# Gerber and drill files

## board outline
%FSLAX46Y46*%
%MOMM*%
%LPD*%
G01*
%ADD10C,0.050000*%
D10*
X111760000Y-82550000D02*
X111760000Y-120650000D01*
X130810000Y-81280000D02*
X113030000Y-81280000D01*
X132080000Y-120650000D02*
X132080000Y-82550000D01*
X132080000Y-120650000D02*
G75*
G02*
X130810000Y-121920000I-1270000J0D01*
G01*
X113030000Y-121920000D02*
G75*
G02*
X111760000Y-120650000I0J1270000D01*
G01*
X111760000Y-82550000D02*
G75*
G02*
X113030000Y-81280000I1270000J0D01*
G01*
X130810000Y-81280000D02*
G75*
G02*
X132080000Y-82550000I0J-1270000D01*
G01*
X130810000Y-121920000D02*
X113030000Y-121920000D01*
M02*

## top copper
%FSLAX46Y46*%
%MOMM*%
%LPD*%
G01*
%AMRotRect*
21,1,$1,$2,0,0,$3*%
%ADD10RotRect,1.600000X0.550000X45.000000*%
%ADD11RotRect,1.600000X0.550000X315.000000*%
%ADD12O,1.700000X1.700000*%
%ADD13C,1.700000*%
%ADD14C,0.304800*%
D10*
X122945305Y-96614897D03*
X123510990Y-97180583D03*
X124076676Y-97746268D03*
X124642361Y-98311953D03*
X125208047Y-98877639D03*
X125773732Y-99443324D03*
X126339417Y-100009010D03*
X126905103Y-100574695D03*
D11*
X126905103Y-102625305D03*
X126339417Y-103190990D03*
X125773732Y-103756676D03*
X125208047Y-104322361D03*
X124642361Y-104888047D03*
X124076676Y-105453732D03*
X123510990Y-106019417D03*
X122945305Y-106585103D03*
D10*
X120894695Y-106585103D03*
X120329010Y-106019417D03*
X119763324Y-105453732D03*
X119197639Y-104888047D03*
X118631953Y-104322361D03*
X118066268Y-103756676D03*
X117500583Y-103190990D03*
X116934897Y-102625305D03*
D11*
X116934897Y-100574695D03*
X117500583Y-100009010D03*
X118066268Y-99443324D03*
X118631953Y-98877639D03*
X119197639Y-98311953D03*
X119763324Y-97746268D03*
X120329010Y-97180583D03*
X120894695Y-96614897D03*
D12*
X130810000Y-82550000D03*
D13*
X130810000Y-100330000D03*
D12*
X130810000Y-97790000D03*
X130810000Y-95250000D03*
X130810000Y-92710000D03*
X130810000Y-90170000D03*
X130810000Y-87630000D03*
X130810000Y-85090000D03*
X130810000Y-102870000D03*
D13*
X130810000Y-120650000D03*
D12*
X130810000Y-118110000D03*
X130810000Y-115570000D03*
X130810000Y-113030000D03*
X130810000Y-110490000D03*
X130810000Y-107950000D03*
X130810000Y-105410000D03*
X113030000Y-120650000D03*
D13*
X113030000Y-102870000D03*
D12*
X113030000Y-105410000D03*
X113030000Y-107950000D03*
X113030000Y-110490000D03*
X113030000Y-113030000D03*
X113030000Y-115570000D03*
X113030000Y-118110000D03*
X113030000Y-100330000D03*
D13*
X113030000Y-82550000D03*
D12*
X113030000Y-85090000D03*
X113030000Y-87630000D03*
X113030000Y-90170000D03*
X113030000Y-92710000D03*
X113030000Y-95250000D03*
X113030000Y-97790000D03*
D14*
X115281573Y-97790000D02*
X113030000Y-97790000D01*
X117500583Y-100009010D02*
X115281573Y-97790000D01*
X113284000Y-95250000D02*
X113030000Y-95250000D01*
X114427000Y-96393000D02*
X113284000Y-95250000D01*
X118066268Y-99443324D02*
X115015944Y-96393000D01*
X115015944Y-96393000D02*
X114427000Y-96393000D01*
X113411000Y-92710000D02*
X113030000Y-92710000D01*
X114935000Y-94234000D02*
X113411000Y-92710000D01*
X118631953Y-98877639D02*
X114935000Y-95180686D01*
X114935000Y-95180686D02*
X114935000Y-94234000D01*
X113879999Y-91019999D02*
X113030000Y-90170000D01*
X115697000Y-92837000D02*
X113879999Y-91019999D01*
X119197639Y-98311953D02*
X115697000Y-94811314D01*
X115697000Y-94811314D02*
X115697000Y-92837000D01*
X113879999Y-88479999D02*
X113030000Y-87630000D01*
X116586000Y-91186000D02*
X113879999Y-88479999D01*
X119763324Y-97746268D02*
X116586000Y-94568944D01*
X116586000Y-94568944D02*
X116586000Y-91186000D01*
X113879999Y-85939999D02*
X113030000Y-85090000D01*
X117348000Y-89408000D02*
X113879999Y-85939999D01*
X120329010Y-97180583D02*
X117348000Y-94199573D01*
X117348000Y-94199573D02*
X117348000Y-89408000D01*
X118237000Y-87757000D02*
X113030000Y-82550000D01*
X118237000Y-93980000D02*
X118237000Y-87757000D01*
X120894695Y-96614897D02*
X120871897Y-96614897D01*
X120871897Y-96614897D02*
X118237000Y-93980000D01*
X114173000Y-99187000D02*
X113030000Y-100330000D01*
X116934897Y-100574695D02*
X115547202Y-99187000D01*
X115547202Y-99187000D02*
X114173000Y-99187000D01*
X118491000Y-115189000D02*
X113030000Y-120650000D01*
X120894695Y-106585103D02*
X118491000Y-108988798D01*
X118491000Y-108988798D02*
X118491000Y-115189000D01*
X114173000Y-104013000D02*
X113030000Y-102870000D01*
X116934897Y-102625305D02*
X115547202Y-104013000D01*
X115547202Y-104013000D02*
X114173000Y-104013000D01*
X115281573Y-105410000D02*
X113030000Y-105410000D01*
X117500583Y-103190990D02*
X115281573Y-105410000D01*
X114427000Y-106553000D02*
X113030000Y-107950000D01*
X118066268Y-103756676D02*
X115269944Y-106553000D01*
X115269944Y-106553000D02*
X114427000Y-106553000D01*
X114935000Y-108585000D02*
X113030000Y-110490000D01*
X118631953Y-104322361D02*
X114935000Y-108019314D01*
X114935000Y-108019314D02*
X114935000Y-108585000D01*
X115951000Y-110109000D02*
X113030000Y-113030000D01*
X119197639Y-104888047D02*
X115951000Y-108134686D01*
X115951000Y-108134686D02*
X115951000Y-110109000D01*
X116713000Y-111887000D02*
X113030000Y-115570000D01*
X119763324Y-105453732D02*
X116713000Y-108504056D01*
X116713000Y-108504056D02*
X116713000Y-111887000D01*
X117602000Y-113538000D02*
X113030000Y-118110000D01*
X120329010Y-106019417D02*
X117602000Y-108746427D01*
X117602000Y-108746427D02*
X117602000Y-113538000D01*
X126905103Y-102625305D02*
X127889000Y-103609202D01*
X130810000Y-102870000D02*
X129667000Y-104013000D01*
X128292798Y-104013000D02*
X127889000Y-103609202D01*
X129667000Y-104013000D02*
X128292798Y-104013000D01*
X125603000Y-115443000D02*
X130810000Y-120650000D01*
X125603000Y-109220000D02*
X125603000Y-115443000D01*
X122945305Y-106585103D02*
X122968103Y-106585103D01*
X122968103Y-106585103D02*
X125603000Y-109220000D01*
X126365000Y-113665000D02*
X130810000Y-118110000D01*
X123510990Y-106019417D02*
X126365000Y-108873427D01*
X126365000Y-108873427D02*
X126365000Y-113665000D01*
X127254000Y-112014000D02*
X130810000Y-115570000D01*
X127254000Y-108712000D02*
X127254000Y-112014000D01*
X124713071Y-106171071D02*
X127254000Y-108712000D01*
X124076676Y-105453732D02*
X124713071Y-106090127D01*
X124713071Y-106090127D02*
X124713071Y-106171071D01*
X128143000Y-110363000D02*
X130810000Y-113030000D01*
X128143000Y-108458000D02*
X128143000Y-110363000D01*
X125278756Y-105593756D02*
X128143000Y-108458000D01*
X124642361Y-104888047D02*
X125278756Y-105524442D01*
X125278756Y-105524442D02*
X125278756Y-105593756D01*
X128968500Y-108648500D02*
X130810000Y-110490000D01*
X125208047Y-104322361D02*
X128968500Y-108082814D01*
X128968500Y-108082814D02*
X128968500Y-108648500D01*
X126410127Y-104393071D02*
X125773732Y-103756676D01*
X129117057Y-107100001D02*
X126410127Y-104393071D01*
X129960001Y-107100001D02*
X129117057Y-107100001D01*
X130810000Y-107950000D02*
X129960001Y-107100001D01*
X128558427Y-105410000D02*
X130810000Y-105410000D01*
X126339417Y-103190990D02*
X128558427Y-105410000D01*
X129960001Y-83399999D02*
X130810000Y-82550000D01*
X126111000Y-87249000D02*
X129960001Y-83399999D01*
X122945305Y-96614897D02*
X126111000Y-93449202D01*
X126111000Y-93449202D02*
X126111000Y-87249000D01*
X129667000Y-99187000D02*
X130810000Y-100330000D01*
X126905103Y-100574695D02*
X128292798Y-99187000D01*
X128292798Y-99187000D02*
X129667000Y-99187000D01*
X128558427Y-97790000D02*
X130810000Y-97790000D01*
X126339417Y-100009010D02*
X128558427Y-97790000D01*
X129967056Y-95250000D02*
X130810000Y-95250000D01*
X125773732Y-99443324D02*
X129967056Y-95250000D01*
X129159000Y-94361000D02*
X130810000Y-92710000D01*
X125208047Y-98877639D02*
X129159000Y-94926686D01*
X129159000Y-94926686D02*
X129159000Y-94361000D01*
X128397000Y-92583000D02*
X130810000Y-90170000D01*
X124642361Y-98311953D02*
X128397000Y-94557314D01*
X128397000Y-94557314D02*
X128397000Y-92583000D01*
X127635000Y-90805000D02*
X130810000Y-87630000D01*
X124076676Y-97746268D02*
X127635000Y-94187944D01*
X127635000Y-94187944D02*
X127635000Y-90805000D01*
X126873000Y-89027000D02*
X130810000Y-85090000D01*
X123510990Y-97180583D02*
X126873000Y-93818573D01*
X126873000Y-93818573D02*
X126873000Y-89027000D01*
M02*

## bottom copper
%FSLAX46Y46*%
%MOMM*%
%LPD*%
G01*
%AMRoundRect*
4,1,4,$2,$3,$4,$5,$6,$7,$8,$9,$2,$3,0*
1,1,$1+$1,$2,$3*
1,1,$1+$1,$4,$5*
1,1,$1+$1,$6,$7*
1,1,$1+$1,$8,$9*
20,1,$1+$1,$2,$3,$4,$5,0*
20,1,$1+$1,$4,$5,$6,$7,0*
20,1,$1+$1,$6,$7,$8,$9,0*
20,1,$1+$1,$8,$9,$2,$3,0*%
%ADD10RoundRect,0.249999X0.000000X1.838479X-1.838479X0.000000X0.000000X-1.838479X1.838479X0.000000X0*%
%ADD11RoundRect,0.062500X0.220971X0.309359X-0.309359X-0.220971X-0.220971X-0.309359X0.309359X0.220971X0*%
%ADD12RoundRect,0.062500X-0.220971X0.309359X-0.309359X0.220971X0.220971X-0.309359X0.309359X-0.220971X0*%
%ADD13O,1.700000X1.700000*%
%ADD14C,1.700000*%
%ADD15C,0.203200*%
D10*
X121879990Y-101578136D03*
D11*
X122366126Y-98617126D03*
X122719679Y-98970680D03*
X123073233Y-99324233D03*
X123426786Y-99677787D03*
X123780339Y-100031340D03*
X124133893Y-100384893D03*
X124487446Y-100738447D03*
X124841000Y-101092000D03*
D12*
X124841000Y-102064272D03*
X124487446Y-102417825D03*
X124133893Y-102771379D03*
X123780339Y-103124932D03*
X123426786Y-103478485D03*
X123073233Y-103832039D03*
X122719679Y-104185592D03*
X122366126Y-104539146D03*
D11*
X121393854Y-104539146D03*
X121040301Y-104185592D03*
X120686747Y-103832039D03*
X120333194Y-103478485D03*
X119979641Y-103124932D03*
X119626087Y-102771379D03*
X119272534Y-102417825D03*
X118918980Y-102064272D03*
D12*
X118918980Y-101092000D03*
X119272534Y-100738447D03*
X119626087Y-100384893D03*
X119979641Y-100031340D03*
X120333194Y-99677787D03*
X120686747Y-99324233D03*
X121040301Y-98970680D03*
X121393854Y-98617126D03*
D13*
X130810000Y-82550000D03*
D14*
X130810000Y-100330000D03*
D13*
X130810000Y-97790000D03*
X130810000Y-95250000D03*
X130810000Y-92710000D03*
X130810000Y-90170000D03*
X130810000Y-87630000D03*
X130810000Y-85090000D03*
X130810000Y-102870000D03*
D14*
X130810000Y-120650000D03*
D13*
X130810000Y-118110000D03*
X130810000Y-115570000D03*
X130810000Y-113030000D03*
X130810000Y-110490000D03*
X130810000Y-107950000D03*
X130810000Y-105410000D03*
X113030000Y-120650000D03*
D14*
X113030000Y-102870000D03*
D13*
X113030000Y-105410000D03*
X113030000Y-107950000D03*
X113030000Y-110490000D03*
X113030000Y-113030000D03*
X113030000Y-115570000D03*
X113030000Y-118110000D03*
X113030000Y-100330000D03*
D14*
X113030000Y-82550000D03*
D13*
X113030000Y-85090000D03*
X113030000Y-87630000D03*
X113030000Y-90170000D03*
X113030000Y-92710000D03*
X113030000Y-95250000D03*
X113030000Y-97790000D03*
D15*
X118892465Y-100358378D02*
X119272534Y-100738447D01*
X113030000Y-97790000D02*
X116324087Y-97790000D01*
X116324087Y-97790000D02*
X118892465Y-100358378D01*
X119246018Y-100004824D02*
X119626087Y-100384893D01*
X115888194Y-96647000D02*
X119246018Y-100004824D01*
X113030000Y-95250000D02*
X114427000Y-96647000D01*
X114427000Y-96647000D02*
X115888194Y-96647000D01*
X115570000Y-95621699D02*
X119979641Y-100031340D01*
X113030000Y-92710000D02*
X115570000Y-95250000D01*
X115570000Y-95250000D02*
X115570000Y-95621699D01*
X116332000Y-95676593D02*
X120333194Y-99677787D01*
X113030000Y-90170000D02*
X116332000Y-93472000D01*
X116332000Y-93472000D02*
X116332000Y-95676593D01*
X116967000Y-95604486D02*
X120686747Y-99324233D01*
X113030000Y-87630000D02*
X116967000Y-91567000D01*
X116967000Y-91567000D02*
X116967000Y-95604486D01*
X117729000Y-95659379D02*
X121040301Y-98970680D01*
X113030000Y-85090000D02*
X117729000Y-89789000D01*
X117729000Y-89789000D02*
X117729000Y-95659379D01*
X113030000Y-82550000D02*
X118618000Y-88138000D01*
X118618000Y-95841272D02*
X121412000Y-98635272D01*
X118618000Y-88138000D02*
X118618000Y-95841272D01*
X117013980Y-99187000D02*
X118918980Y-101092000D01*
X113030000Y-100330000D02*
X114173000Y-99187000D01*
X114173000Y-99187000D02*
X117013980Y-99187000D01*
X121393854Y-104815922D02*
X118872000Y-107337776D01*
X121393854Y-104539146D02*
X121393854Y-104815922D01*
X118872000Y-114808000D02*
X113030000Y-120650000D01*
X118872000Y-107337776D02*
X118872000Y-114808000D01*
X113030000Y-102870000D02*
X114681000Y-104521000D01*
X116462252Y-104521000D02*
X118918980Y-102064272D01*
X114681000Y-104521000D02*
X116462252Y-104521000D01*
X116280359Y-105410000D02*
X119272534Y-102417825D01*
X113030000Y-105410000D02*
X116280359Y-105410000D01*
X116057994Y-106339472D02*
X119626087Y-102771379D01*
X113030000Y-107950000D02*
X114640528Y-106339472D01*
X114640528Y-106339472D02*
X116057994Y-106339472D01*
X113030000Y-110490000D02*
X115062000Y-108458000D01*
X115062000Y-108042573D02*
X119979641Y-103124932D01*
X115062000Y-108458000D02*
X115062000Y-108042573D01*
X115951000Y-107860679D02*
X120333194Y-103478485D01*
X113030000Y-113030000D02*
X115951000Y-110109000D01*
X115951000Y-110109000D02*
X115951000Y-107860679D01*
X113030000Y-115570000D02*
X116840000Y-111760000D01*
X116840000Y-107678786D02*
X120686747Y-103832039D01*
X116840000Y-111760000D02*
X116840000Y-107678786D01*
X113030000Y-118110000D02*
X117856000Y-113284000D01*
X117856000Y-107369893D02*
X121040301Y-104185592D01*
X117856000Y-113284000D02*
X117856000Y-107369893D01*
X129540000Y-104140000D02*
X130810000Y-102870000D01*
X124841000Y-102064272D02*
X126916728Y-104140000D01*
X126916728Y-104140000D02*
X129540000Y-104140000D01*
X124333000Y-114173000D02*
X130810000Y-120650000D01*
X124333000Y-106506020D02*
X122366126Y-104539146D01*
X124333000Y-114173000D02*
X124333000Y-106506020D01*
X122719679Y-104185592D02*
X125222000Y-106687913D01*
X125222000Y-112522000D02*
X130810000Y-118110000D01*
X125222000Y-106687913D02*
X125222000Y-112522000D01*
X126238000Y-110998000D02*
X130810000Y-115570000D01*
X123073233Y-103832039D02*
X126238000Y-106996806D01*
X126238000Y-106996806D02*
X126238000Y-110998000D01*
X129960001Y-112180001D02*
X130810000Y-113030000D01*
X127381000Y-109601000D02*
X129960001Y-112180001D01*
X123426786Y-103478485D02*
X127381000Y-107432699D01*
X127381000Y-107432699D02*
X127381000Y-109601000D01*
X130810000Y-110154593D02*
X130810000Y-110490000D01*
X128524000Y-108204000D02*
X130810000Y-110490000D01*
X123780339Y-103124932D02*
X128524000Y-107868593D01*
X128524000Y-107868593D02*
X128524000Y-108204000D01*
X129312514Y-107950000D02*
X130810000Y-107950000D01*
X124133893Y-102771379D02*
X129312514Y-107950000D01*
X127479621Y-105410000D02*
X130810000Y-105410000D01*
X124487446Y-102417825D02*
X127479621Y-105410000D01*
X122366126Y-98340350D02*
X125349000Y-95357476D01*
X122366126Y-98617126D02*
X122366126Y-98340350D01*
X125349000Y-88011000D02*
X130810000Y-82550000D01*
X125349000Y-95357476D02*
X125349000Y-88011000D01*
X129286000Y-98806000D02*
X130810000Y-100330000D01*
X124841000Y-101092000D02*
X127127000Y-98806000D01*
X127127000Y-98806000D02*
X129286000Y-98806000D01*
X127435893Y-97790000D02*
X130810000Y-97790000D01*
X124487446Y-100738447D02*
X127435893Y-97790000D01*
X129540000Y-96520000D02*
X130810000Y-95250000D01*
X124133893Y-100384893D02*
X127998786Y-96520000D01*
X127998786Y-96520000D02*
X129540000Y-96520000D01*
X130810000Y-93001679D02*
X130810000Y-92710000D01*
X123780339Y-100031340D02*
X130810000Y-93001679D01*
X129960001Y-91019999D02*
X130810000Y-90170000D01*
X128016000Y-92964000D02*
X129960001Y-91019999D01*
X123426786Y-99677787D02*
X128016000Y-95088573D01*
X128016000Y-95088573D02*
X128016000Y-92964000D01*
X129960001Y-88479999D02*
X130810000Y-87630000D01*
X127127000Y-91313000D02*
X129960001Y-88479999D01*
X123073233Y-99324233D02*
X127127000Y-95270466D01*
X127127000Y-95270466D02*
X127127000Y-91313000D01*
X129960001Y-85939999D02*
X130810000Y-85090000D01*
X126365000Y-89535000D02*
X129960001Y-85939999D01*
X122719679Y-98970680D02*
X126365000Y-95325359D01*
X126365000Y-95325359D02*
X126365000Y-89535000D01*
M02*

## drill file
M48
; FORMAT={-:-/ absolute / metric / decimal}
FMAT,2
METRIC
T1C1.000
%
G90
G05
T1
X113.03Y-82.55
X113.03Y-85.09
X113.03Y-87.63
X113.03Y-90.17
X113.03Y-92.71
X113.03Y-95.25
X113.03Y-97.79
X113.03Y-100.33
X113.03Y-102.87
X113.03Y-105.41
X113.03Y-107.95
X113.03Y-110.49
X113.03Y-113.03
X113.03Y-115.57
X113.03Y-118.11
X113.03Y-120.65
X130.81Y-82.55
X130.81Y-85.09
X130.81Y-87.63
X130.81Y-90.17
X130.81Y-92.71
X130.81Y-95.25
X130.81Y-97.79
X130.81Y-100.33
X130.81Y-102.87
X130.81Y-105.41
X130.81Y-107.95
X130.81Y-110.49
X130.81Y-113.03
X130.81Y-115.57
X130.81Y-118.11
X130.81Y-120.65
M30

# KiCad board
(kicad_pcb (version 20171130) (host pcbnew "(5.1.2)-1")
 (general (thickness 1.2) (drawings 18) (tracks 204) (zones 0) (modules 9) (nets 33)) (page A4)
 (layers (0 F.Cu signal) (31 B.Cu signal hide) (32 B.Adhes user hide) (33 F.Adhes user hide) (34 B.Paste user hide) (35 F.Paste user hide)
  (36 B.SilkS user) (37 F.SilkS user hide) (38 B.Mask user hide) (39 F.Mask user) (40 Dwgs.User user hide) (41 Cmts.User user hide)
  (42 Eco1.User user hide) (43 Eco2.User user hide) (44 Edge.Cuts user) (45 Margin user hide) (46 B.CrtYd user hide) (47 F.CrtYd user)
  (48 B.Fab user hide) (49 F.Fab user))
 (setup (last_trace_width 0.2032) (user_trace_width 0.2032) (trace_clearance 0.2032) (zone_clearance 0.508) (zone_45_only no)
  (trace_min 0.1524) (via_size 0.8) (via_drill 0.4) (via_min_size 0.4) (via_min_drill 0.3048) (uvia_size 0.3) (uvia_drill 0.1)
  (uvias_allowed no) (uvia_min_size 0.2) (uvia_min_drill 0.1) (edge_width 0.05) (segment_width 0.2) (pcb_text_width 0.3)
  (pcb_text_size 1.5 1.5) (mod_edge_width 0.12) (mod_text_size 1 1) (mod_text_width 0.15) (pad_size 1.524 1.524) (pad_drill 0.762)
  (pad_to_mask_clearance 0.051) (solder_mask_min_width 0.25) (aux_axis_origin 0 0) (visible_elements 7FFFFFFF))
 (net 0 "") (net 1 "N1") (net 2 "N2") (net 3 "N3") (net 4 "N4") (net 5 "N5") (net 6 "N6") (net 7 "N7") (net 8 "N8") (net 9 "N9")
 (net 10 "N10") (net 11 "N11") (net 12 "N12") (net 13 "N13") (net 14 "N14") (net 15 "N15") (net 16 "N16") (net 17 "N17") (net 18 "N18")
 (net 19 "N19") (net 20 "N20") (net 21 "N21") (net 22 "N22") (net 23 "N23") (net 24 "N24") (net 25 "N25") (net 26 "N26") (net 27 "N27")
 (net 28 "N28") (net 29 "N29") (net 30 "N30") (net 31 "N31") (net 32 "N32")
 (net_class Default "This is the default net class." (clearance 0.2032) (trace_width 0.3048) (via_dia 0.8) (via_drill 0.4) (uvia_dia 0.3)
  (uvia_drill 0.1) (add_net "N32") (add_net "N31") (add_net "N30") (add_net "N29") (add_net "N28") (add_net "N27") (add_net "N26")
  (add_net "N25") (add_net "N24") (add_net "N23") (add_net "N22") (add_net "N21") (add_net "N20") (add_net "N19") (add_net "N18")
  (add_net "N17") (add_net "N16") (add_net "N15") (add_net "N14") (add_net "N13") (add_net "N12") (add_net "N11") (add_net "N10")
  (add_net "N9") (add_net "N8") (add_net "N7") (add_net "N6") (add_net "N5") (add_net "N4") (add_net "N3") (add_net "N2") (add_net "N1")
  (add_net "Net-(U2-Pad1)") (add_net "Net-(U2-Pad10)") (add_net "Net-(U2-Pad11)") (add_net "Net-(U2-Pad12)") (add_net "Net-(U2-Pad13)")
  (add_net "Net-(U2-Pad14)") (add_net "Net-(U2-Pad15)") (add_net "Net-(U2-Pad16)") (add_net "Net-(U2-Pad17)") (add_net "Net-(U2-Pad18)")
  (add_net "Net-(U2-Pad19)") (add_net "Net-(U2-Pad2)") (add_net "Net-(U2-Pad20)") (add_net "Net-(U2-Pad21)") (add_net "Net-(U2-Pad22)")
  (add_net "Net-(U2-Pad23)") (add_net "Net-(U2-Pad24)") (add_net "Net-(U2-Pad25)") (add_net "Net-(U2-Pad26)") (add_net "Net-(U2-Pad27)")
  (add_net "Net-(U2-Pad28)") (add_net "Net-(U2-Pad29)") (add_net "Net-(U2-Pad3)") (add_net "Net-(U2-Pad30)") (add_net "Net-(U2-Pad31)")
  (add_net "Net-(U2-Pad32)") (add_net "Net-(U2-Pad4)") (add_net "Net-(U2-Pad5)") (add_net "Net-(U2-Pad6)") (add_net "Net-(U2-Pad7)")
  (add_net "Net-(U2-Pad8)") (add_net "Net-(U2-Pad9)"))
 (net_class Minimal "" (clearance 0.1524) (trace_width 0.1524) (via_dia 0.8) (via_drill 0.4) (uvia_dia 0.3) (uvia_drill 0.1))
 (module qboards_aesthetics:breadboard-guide (layer F.Cu) (at 97.79 90.17)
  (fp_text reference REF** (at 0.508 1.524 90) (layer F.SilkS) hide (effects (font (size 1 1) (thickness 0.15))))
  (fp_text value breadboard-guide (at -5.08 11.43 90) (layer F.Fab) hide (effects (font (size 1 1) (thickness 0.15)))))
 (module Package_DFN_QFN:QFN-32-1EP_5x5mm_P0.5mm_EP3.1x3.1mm (layer B.Cu) (at 121.87999 101.578136 225)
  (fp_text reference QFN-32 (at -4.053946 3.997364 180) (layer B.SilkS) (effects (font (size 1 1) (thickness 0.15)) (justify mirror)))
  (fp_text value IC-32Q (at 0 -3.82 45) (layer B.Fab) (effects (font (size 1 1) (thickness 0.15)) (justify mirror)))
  (pad 33 smd roundrect (at 0 0 225) (size 3.1 3.1) (layers B.Cu B.Mask) (roundrect_rratio 0.08064499999999999))
  (pad "" smd roundrect (at -1.03 1.03 225) (size 0.83 0.83) (layers B.Paste) (roundrect_rratio 0.25))
  (pad "" smd roundrect (at -1.03 0 225) (size 0.83 0.83) (layers B.Paste) (roundrect_rratio 0.25))
  (pad "" smd roundrect (at -1.03 -1.03 225) (size 0.83 0.83) (layers B.Paste) (roundrect_rratio 0.25))
  (pad "" smd roundrect (at 0 1.03 225) (size 0.83 0.83) (layers B.Paste) (roundrect_rratio 0.25))
  (pad "" smd roundrect (at 0 0 225) (size 0.83 0.83) (layers B.Paste) (roundrect_rratio 0.25))
  (pad "" smd roundrect (at 0 -1.03 225) (size 0.83 0.83) (layers B.Paste) (roundrect_rratio 0.25))
  (pad "" smd roundrect (at 1.03 1.03 225) (size 0.83 0.83) (layers B.Paste) (roundrect_rratio 0.25))
  (pad "" smd roundrect (at 1.03 0 225) (size 0.83 0.83) (layers B.Paste) (roundrect_rratio 0.25))
  (pad "" smd roundrect (at 1.03 -1.03 225) (size 0.83 0.83) (layers B.Paste) (roundrect_rratio 0.25))
  (pad 1 smd roundrect (at -2.4375 1.75 225) (size 0.875 0.25) (layers B.Cu B.Paste B.Mask) (roundrect_rratio 0.25) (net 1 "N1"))
  (pad 2 smd roundrect (at -2.4375 1.25 225) (size 0.875 0.25) (layers B.Cu B.Paste B.Mask) (roundrect_rratio 0.25) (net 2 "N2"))
  (pad 3 smd roundrect (at -2.4375 0.75 225) (size 0.875 0.25) (layers B.Cu B.Paste B.Mask) (roundrect_rratio 0.25) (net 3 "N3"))
  (pad 4 smd roundrect (at -2.4375 0.25 225) (size 0.875 0.25) (layers B.Cu B.Paste B.Mask) (roundrect_rratio 0.25) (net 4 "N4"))
  (pad 5 smd roundrect (at -2.4375 -0.25 225) (size 0.875 0.25) (layers B.Cu B.Paste B.Mask) (roundrect_rratio 0.25) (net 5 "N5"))
  (pad 6 smd roundrect (at -2.4375 -0.75 225) (size 0.875 0.25) (layers B.Cu B.Paste B.Mask) (roundrect_rratio 0.25) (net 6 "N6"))
  (pad 7 smd roundrect (at -2.4375 -1.25 225) (size 0.875 0.25) (layers B.Cu B.Paste B.Mask) (roundrect_rratio 0.25) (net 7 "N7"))
  (pad 8 smd roundrect (at -2.4375 -1.75 225) (size 0.875 0.25) (layers B.Cu B.Paste B.Mask) (roundrect_rratio 0.25) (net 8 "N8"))
  (pad 9 smd roundrect (at -1.75 -2.4375 225) (size 0.25 0.875) (layers B.Cu B.Paste B.Mask) (roundrect_rratio 0.25) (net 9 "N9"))
  (pad 10 smd roundrect (at -1.25 -2.4375 225) (size 0.25 0.875) (layers B.Cu B.Paste B.Mask) (roundrect_rratio 0.25) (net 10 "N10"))
  (pad 11 smd roundrect (at -0.75 -2.4375 225) (size 0.25 0.875) (layers B.Cu B.Paste B.Mask) (roundrect_rratio 0.25) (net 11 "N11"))
  (pad 12 smd roundrect (at -0.25 -2.4375 225) (size 0.25 0.875) (layers B.Cu B.Paste B.Mask) (roundrect_rratio 0.25) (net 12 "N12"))
  (pad 13 smd roundrect (at 0.25 -2.4375 225) (size 0.25 0.875) (layers B.Cu B.Paste B.Mask) (roundrect_rratio 0.25) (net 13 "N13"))
  (pad 14 smd roundrect (at 0.75 -2.4375 225) (size 0.25 0.875) (layers B.Cu B.Paste B.Mask) (roundrect_rratio 0.25) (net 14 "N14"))
  (pad 15 smd roundrect (at 1.25 -2.4375 225) (size 0.25 0.875) (layers B.Cu B.Paste B.Mask) (roundrect_rratio 0.25) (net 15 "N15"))
  (pad 16 smd roundrect (at 1.75 -2.4375 225) (size 0.25 0.875) (layers B.Cu B.Paste B.Mask) (roundrect_rratio 0.25) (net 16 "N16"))
  (pad 17 smd roundrect (at 2.4375 -1.75 225) (size 0.875 0.25) (layers B.Cu B.Paste B.Mask) (roundrect_rratio 0.25) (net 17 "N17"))
  (pad 18 smd roundrect (at 2.4375 -1.25 225) (size 0.875 0.25) (layers B.Cu B.Paste B.Mask) (roundrect_rratio 0.25) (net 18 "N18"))
  (pad 19 smd roundrect (at 2.4375 -0.75 225) (size 0.875 0.25) (layers B.Cu B.Paste B.Mask) (roundrect_rratio 0.25) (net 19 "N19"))
  (pad 20 smd roundrect (at 2.4375 -0.25 225) (size 0.875 0.25) (layers B.Cu B.Paste B.Mask) (roundrect_rratio 0.25) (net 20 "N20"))
  (pad 21 smd roundrect (at 2.4375 0.25 225) (size 0.875 0.25) (layers B.Cu B.Paste B.Mask) (roundrect_rratio 0.25) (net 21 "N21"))
  (pad 22 smd roundrect (at 2.4375 0.75 225) (size 0.875 0.25) (layers B.Cu B.Paste B.Mask) (roundrect_rratio 0.25) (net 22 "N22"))
  (pad 23 smd roundrect (at 2.4375 1.25 225) (size 0.875 0.25) (layers B.Cu B.Paste B.Mask) (roundrect_rratio 0.25) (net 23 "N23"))
  (pad 24 smd roundrect (at 2.4375 1.75 225) (size 0.875 0.25) (layers B.Cu B.Paste B.Mask) (roundrect_rratio 0.25) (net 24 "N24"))
  (pad 25 smd roundrect (at 1.75 2.4375 225) (size 0.25 0.875) (layers B.Cu B.Paste B.Mask) (roundrect_rratio 0.25) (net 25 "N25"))
  (pad 26 smd roundrect (at 1.25 2.4375 225) (size 0.25 0.875) (layers B.Cu B.Paste B.Mask) (roundrect_rratio 0.25) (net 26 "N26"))
  (pad 27 smd roundrect (at 0.75 2.4375 225) (size 0.25 0.875) (layers B.Cu B.Paste B.Mask) (roundrect_rratio 0.25) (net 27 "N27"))
  (pad 28 smd roundrect (at 0.25 2.4375 225) (size 0.25 0.875) (layers B.Cu B.Paste B.Mask) (roundrect_rratio 0.25) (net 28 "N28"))
  (pad 29 smd roundrect (at -0.25 2.4375 225) (size 0.25 0.875) (layers B.Cu B.Paste B.Mask) (roundrect_rratio 0.25) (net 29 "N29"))
  (pad 30 smd roundrect (at -0.75 2.4375 225) (size 0.25 0.875) (layers B.Cu B.Paste B.Mask) (roundrect_rratio 0.25) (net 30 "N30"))
  (pad 31 smd roundrect (at -1.25 2.4375 225) (size 0.25 0.875) (layers B.Cu B.Paste B.Mask) (roundrect_rratio 0.25) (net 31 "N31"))
  (pad 32 smd roundrect (at -1.75 2.4375 225) (size 0.25 0.875) (layers B.Cu B.Paste B.Mask) (roundrect_rratio 0.25) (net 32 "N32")))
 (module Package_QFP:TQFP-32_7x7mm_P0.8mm (layer F.Cu) (at 121.92 101.6 315)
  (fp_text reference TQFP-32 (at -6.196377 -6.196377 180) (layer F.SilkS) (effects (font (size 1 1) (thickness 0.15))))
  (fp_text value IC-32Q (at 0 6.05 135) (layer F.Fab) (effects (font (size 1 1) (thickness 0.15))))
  (pad 32 smd rect (at -2.8 -4.25 45) (size 1.6 0.55) (layers F.Cu F.Paste F.Mask) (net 1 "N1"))
  (pad 31 smd rect (at -2 -4.25 45) (size 1.6 0.55) (layers F.Cu F.Paste F.Mask) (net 2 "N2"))
  (pad 30 smd rect (at -1.2 -4.25 45) (size 1.6 0.55) (layers F.Cu F.Paste F.Mask) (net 3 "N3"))
  (pad 29 smd rect (at -0.4 -4.25 45) (size 1.6 0.55) (layers F.Cu F.Paste F.Mask) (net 4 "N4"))
  (pad 28 smd rect (at 0.4 -4.25 45) (size 1.6 0.55) (layers F.Cu F.Paste F.Mask) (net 5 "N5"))
  (pad 27 smd rect (at 1.2 -4.25 45) (size 1.6 0.55) (layers F.Cu F.Paste F.Mask) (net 6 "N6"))
  (pad 26 smd rect (at 2 -4.25 45) (size 1.6 0.55) (layers F.Cu F.Paste F.Mask) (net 7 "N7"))
  (pad 25 smd rect (at 2.8 -4.25 45) (size 1.6 0.55) (layers F.Cu F.Paste F.Mask) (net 8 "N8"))
  (pad 24 smd rect (at 4.25 -2.8 315) (size 1.6 0.55) (layers F.Cu F.Paste F.Mask) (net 9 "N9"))
  (pad 23 smd rect (at 4.25 -2 315) (size 1.6 0.55) (layers F.Cu F.Paste F.Mask) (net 10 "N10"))
  (pad 22 smd rect (at 4.25 -1.2 315) (size 1.6 0.55) (layers F.Cu F.Paste F.Mask) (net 11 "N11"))
  (pad 21 smd rect (at 4.25 -0.4 315) (size 1.6 0.55) (layers F.Cu F.Paste F.Mask) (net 12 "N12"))
  (pad 20 smd rect (at 4.25 0.4 315) (size 1.6 0.55) (layers F.Cu F.Paste F.Mask) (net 13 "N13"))
  (pad 19 smd rect (at 4.25 1.2 315) (size 1.6 0.55) (layers F.Cu F.Paste F.Mask) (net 14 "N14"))
  (pad 18 smd rect (at 4.25 2 315) (size 1.6 0.55) (layers F.Cu F.Paste F.Mask) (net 15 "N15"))
  (pad 17 smd rect (at 4.25 2.8 315) (size 1.6 0.55) (layers F.Cu F.Paste F.Mask) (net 16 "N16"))
  (pad 16 smd rect (at 2.8 4.25 45) (size 1.6 0.55) (layers F.Cu F.Paste F.Mask) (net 17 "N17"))
  (pad 15 smd rect (at 2 4.25 45) (size 1.6 0.55) (layers F.Cu F.Paste F.Mask) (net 18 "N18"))
  (pad 14 smd rect (at 1.2 4.25 45) (size 1.6 0.55) (layers F.Cu F.Paste F.Mask) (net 19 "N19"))
  (pad 13 smd rect (at 0.4 4.25 45) (size 1.6 0.55) (layers F.Cu F.Paste F.Mask) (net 20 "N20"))
  (pad 12 smd rect (at -0.4 4.25 45) (size 1.6 0.55) (layers F.Cu F.Paste F.Mask) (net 21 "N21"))
  (pad 11 smd rect (at -1.2 4.25 45) (size 1.6 0.55) (layers F.Cu F.Paste F.Mask) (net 22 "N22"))
  (pad 10 smd rect (at -2 4.25 45) (size 1.6 0.55) (layers F.Cu F.Paste F.Mask) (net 23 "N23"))
  (pad 9 smd rect (at -2.8 4.25 45) (size 1.6 0.55) (layers F.Cu F.Paste F.Mask) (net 24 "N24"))
  (pad 8 smd rect (at -4.25 2.8 315) (size 1.6 0.55) (layers F.Cu F.Paste F.Mask) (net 25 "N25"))
  (pad 7 smd rect (at -4.25 2 315) (size 1.6 0.55) (layers F.Cu F.Paste F.Mask) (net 26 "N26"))
  (pad 6 smd rect (at -4.25 1.2 315) (size 1.6 0.55) (layers F.Cu F.Paste F.Mask) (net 27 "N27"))
  (pad 5 smd rect (at -4.25 0.4 315) (size 1.6 0.55) (layers F.Cu F.Paste F.Mask) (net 28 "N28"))
  (pad 4 smd rect (at -4.25 -0.4 315) (size 1.6 0.55) (layers F.Cu F.Paste F.Mask) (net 29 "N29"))
  (pad 3 smd rect (at -4.25 -1.2 315) (size 1.6 0.55) (layers F.Cu F.Paste F.Mask) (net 30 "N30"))
  (pad 2 smd rect (at -4.25 -2 315) (size 1.6 0.55) (layers F.Cu F.Paste F.Mask) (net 31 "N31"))
  (pad 1 smd rect (at -4.25 -2.8 315) (size 1.6 0.55) (layers F.Cu F.Paste F.Mask) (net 32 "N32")))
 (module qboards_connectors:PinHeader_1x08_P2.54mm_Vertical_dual (layer F.Cu) (at 130.81 100.33 180)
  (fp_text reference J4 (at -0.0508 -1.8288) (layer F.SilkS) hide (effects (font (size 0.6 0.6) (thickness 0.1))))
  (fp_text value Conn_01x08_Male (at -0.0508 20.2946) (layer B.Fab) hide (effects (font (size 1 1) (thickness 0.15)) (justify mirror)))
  (pad 8 thru_hole oval (at 0 17.78 180) (size 1.7 1.7) (drill 1) (layers *.Cu *.Mask) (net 1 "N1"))
  (pad 1 thru_hole circle (at 0 0 180) (size 1.7 1.7) (drill 1) (layers *.Cu *.Mask) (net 8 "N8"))
  (pad 2 thru_hole oval (at 0 2.54 180) (size 1.7 1.7) (drill 1) (layers *.Cu *.Mask) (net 7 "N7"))
  (pad 3 thru_hole oval (at 0 5.08 180) (size 1.7 1.7) (drill 1) (layers *.Cu *.Mask) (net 6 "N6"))
  (pad 4 thru_hole oval (at 0 7.62 180) (size 1.7 1.7) (drill 1) (layers *.Cu *.Mask) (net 5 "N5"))
  (pad 5 thru_hole oval (at 0 10.16 180) (size 1.7 1.7) (drill 1) (layers *.Cu *.Mask) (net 4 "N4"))
  (pad 6 thru_hole oval (at 0 12.7 180) (size 1.7 1.7) (drill 1) (layers *.Cu *.Mask) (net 3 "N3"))
  (pad 7 thru_hole oval (at 0 15.24 180) (size 1.7 1.7) (drill 1) (layers *.Cu *.Mask) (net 2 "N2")))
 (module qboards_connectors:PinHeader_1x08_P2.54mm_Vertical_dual (layer F.Cu) (at 130.81 120.65 180)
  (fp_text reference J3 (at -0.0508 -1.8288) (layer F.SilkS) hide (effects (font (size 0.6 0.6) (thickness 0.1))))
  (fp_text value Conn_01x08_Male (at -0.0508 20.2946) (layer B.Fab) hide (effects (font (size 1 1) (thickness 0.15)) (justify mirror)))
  (pad 8 thru_hole oval (at 0 17.78 180) (size 1.7 1.7) (drill 1) (layers *.Cu *.Mask) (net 9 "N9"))
  (pad 1 thru_hole circle (at 0 0 180) (size 1.7 1.7) (drill 1) (layers *.Cu *.Mask) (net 16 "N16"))
  (pad 2 thru_hole oval (at 0 2.54 180) (size 1.7 1.7) (drill 1) (layers *.Cu *.Mask) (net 15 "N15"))
  (pad 3 thru_hole oval (at 0 5.08 180) (size 1.7 1.7) (drill 1) (layers *.Cu *.Mask) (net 14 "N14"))
  (pad 4 thru_hole oval (at 0 7.62 180) (size 1.7 1.7) (drill 1) (layers *.Cu *.Mask) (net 13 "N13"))
  (pad 5 thru_hole oval (at 0 10.16 180) (size 1.7 1.7) (drill 1) (layers *.Cu *.Mask) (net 12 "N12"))
  (pad 6 thru_hole oval (at 0 12.7 180) (size 1.7 1.7) (drill 1) (layers *.Cu *.Mask) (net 11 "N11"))
  (pad 7 thru_hole oval (at 0 15.24 180) (size 1.7 1.7) (drill 1) (layers *.Cu *.Mask) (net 10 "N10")))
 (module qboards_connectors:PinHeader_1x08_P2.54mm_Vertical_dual (layer F.Cu) (at 113.03 102.87)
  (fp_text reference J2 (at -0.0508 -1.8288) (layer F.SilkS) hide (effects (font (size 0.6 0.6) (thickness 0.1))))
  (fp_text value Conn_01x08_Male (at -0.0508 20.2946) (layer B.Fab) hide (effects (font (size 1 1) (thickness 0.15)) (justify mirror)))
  (pad 8 thru_hole oval (at 0 17.78) (size 1.7 1.7) (drill 1) (layers *.Cu *.Mask) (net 17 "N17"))
  (pad 1 thru_hole circle (at 0 0) (size 1.7 1.7) (drill 1) (layers *.Cu *.Mask) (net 24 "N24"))
  (pad 2 thru_hole oval (at 0 2.54) (size 1.7 1.7) (drill 1) (layers *.Cu *.Mask) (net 23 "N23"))
  (pad 3 thru_hole oval (at 0 5.08) (size 1.7 1.7) (drill 1) (layers *.Cu *.Mask) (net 22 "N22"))
  (pad 4 thru_hole oval (at 0 7.62) (size 1.7 1.7) (drill 1) (layers *.Cu *.Mask) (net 21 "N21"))
  (pad 5 thru_hole oval (at 0 10.16) (size 1.7 1.7) (drill 1) (layers *.Cu *.Mask) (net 20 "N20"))
  (pad 6 thru_hole oval (at 0 12.7) (size 1.7 1.7) (drill 1) (layers *.Cu *.Mask) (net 19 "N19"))
  (pad 7 thru_hole oval (at 0 15.24) (size 1.7 1.7) (drill 1) (layers *.Cu *.Mask) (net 18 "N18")))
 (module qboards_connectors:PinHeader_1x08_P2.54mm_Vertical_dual (layer F.Cu) (at 113.03 82.55)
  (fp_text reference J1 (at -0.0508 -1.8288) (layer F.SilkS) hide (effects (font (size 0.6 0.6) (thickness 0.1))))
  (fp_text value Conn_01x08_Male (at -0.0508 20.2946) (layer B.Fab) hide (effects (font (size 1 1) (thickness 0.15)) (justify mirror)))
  (pad 8 thru_hole oval (at 0 17.78) (size 1.7 1.7) (drill 1) (layers *.Cu *.Mask) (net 25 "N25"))
  (pad 1 thru_hole circle (at 0 0) (size 1.7 1.7) (drill 1) (layers *.Cu *.Mask) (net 32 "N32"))
  (pad 2 thru_hole oval (at 0 2.54) (size 1.7 1.7) (drill 1) (layers *.Cu *.Mask) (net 31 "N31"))
  (pad 3 thru_hole oval (at 0 5.08) (size 1.7 1.7) (drill 1) (layers *.Cu *.Mask) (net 30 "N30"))
  (pad 4 thru_hole oval (at 0 7.62) (size 1.7 1.7) (drill 1) (layers *.Cu *.Mask) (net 29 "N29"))
  (pad 5 thru_hole oval (at 0 10.16) (size 1.7 1.7) (drill 1) (layers *.Cu *.Mask) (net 28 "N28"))
  (pad 6 thru_hole oval (at 0 12.7) (size 1.7 1.7) (drill 1) (layers *.Cu *.Mask) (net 27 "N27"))
  (pad 7 thru_hole oval (at 0 15.24) (size 1.7 1.7) (drill 1) (layers *.Cu *.Mask) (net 26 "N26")))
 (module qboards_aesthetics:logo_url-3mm (layer F.Cu) (at 117.602 117.983)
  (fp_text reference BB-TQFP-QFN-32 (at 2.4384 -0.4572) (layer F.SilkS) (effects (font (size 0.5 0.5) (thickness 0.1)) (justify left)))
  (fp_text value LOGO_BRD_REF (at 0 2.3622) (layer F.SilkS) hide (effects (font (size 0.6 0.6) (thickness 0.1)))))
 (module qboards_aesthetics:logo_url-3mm (layer B.Cu) (at 126.492 117.983 180)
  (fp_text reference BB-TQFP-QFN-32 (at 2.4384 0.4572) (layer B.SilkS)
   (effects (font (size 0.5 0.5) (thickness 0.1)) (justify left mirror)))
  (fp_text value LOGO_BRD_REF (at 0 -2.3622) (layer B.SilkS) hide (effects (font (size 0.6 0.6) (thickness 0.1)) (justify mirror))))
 (gr_line (start 111.76 82.55) (end 111.76 120.65) (layer Edge.Cuts) (width 0.05))
 (gr_line (start 130.81 81.28) (end 113.03 81.28) (layer Edge.Cuts) (width 0.05))
 (gr_line (start 132.08 120.65) (end 132.08 82.55) (layer Edge.Cuts) (width 0.05))
 (gr_arc (start 130.81 120.65) (end 130.81 121.92) (angle -90) (layer Edge.Cuts) (width 0.05))
 (gr_arc (start 113.03 120.65) (end 111.76 120.65) (angle -90) (layer Edge.Cuts) (width 0.05))
 (gr_arc (start 113.03 82.55) (end 113.03 81.28) (angle -90) (layer Edge.Cuts) (width 0.05))
 (gr_arc (start 130.81 82.55) (end 132.08 82.55) (angle -90) (layer Edge.Cuts) (width 0.05))
 (gr_line (start 130.81 121.92) (end 113.03 121.92) (layer Edge.Cuts) (width 0.05))
 (segment (start 115.281573 97.79) (end 113.03 97.79) (width 0.3048) (layer F.Cu) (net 26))
 (segment (start 117.500583 100.00901) (end 115.281573 97.79) (width 0.3048) (layer F.Cu) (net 26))
 (segment (start 118.892465 100.358378) (end 119.272534 100.738447) (width 0.2032) (layer B.Cu) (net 26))
 (segment (start 113.03 97.79) (end 116.324087 97.79) (width 0.2032) (layer B.Cu) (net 26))
 (segment (start 116.324087 97.79) (end 118.892465 100.358378) (width 0.2032) (layer B.Cu) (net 26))
 (segment (start 113.284 95.25) (end 113.03 95.25) (width 0.3048) (layer F.Cu) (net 27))
 (segment (start 114.427 96.393) (end 113.284 95.25) (width 0.3048) (layer F.Cu) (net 27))
 (segment (start 118.066268 99.443324) (end 115.015944 96.393) (width 0.3048) (layer F.Cu) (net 27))
 (segment (start 115.015944 96.393) (end 114.427 96.393) (width 0.3048) (layer F.Cu) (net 27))
 (segment (start 119.246018 100.004824) (end 119.626087 100.384893) (width 0.2032) (layer B.Cu) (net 27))
 (segment (start 115.888194 96.647) (end 119.246018 100.004824) (width 0.2032) (layer B.Cu) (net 27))
 (segment (start 113.03 95.25) (end 114.427 96.647) (width 0.2032) (layer B.Cu) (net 27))
 (segment (start 114.427 96.647) (end 115.888194 96.647) (width 0.2032) (layer B.Cu) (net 27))
 (segment (start 113.411 92.71) (end 113.03 92.71) (width 0.3048) (layer F.Cu) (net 28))
 (segment (start 114.935 94.234) (end 113.411 92.71) (width 0.3048) (layer F.Cu) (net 28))
 (segment (start 118.631953 98.877639) (end 114.935 95.180686) (width 0.3048) (layer F.Cu) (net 28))
 (segment (start 114.935 95.180686) (end 114.935 94.234) (width 0.3048) (layer F.Cu) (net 28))
 (segment (start 115.57 95.621699) (end 119.979641 100.03134) (width 0.2032) (layer B.Cu) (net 28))
 (segment (start 113.03 92.71) (end 115.57 95.25) (width 0.2032) (layer B.Cu) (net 28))
 (segment (start 115.57 95.25) (end 115.57 95.621699) (width 0.2032) (layer B.Cu) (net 28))
 (segment (start 113.879999 91.019999) (end 113.03 90.17) (width 0.3048) (layer F.Cu) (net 29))
 (segment (start 115.697 92.837) (end 113.879999 91.019999) (width 0.3048) (layer F.Cu) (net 29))
 (segment (start 119.197639 98.311953) (end 115.697 94.811314) (width 0.3048) (layer F.Cu) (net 29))
 (segment (start 115.697 94.811314) (end 115.697 92.837) (width 0.3048) (layer F.Cu) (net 29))
 (segment (start 116.332 95.676593) (end 120.333194 99.677787) (width 0.2032) (layer B.Cu) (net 29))
 (segment (start 113.03 90.17) (end 116.332 93.472) (width 0.2032) (layer B.Cu) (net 29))
 (segment (start 116.332 93.472) (end 116.332 95.676593) (width 0.2032) (layer B.Cu) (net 29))
 (segment (start 113.879999 88.479999) (end 113.03 87.63) (width 0.3048) (layer F.Cu) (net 30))
 (segment (start 116.586 91.186) (end 113.879999 88.479999) (width 0.3048) (layer F.Cu) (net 30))
 (segment (start 119.763324 97.746268) (end 116.586 94.568944) (width 0.3048) (layer F.Cu) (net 30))
 (segment (start 116.586 94.568944) (end 116.586 91.186) (width 0.3048) (layer F.Cu) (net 30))
 (segment (start 116.967 95.604486) (end 120.686747 99.324233) (width 0.2032) (layer B.Cu) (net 30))
 (segment (start 113.03 87.63) (end 116.967 91.567) (width 0.2032) (layer B.Cu) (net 30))
 (segment (start 116.967 91.567) (end 116.967 95.604486) (width 0.2032) (layer B.Cu) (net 30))
 (segment (start 113.879999 85.939999) (end 113.03 85.09) (width 0.3048) (layer F.Cu) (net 31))
 (segment (start 117.348 89.408) (end 113.879999 85.939999) (width 0.3048) (layer F.Cu) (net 31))
 (segment (start 120.32901 97.180583) (end 117.348 94.199573) (width 0.3048) (layer F.Cu) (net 31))
 (segment (start 117.348 94.199573) (end 117.348 89.408) (width 0.3048) (layer F.Cu) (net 31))
 (segment (start 117.729 95.659379) (end 121.040301 98.97068) (width 0.2032) (layer B.Cu) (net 31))
 (segment (start 113.03 85.09) (end 117.729 89.789) (width 0.2032) (layer B.Cu) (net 31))
 (segment (start 117.729 89.789) (end 117.729 95.659379) (width 0.2032) (layer B.Cu) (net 31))
 (segment (start 118.237 87.757) (end 113.03 82.55) (width 0.3048) (layer F.Cu) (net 32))
 (segment (start 118.237 93.98) (end 118.237 87.757) (width 0.3048) (layer F.Cu) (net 32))
 (segment (start 120.894695 96.614897) (end 120.871897 96.614897) (width 0.3048) (layer F.Cu) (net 32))
 (segment (start 120.871897 96.614897) (end 118.237 93.98) (width 0.3048) (layer F.Cu) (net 32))
 (segment (start 113.03 82.55) (end 118.618 88.138) (width 0.2032) (layer B.Cu) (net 32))
 (segment (start 118.618 95.841272) (end 121.412 98.635272) (width 0.2032) (layer B.Cu) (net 32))
 (segment (start 118.618 88.138) (end 118.618 95.841272) (width 0.2032) (layer B.Cu) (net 32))
 (segment (start 114.173 99.187) (end 113.03 100.33) (width 0.3048) (layer F.Cu) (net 25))
 (segment (start 116.934897 100.574695) (end 115.547202 99.187) (width 0.3048) (layer F.Cu) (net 25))
 (segment (start 115.547202 99.187) (end 114.173 99.187) (width 0.3048) (layer F.Cu) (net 25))
 (segment (start 117.01398 99.187) (end 118.91898 101.092) (width 0.2032) (layer B.Cu) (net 25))
 (segment (start 113.03 100.33) (end 114.173 99.187) (width 0.2032) (layer B.Cu) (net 25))
 (segment (start 114.173 99.187) (end 117.01398 99.187) (width 0.2032) (layer B.Cu) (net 25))
 (segment (start 118.491 115.189) (end 113.03 120.65) (width 0.3048) (layer F.Cu) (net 17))
 (segment (start 120.894695 106.585103) (end 118.491 108.988798) (width 0.3048) (layer F.Cu) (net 17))
 (segment (start 118.491 108.988798) (end 118.491 115.189) (width 0.3048) (layer F.Cu) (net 17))
 (segment (start 121.393854 104.815922) (end 118.872 107.337776) (width 0.2032) (layer B.Cu) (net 17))
 (segment (start 121.393854 104.539146) (end 121.393854 104.815922) (width 0.2032) (layer B.Cu) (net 17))
 (segment (start 118.872 114.808) (end 113.03 120.65) (width 0.2032) (layer B.Cu) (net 17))
 (segment (start 118.872 107.337776) (end 118.872 114.808) (width 0.2032) (layer B.Cu) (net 17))
 (segment (start 114.173 104.013) (end 113.03 102.87) (width 0.3048) (layer F.Cu) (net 24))
 (segment (start 116.934897 102.625305) (end 115.547202 104.013) (width 0.3048) (layer F.Cu) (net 24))
 (segment (start 115.547202 104.013) (end 114.173 104.013) (width 0.3048) (layer F.Cu) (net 24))
 (segment (start 113.03 102.87) (end 114.681 104.521) (width 0.2032) (layer B.Cu) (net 24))
 (segment (start 116.462252 104.521) (end 118.91898 102.064272) (width 0.2032) (layer B.Cu) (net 24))
 (segment (start 114.681 104.521) (end 116.462252 104.521) (width 0.2032) (layer B.Cu) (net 24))
 (segment (start 115.281573 105.41) (end 113.03 105.41) (width 0.3048) (layer F.Cu) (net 23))
 (segment (start 117.500583 103.19099) (end 115.281573 105.41) (width 0.3048) (layer F.Cu) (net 23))
 (segment (start 116.280359 105.41) (end 119.272534 102.417825) (width 0.2032) (layer B.Cu) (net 23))
 (segment (start 113.03 105.41) (end 116.280359 105.41) (width 0.2032) (layer B.Cu) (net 23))
 (segment (start 114.427 106.553) (end 113.03 107.95) (width 0.3048) (layer F.Cu) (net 22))
 (segment (start 118.066268 103.756676) (end 115.269944 106.553) (width 0.3048) (layer F.Cu) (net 22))
 (segment (start 115.269944 106.553) (end 114.427 106.553) (width 0.3048) (layer F.Cu) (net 22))
 (segment (start 116.057994 106.339472) (end 119.626087 102.771379) (width 0.2032) (layer B.Cu) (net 22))
 (segment (start 113.03 107.95) (end 114.640528 106.339472) (width 0.2032) (layer B.Cu) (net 22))
 (segment (start 114.640528 106.339472) (end 116.057994 106.339472) (width 0.2032) (layer B.Cu) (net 22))
 (segment (start 114.935 108.585) (end 113.03 110.49) (width 0.3048) (layer F.Cu) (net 21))
 (segment (start 118.631953 104.322361) (end 114.935 108.019314) (width 0.3048) (layer F.Cu) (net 21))
 (segment (start 114.935 108.019314) (end 114.935 108.585) (width 0.3048) (layer F.Cu) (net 21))
 (segment (start 113.03 110.49) (end 115.062 108.458) (width 0.2032) (layer B.Cu) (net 21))
 (segment (start 115.062 108.042573) (end 119.979641 103.124932) (width 0.2032) (layer B.Cu) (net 21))
 (segment (start 115.062 108.458) (end 115.062 108.042573) (width 0.2032) (layer B.Cu) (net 21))
 (segment (start 115.951 110.109) (end 113.03 113.03) (width 0.3048) (layer F.Cu) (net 20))
 (segment (start 119.197639 104.888047) (end 115.951 108.134686) (width 0.3048) (layer F.Cu) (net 20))
 (segment (start 115.951 108.134686) (end 115.951 110.109) (width 0.3048) (layer F.Cu) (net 20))
 (segment (start 115.951 107.860679) (end 120.333194 103.478485) (width 0.2032) (layer B.Cu) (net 20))
 (segment (start 113.03 113.03) (end 115.951 110.109) (width 0.2032) (layer B.Cu) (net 20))
 (segment (start 115.951 110.109) (end 115.951 107.860679) (width 0.2032) (layer B.Cu) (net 20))
 (segment (start 116.713 111.887) (end 113.03 115.57) (width 0.3048) (layer F.Cu) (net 19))
 (segment (start 119.763324 105.453732) (end 116.713 108.504056) (width 0.3048) (layer F.Cu) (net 19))
 (segment (start 116.713 108.504056) (end 116.713 111.887) (width 0.3048) (layer F.Cu) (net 19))
 (segment (start 113.03 115.57) (end 116.84 111.76) (width 0.2032) (layer B.Cu) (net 19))
 (segment (start 116.84 107.678786) (end 120.686747 103.832039) (width 0.2032) (layer B.Cu) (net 19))
 (segment (start 116.84 111.76) (end 116.84 107.678786) (width 0.2032) (layer B.Cu) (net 19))
 (segment (start 117.602 113.538) (end 113.03 118.11) (width 0.3048) (layer F.Cu) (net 18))
 (segment (start 120.32901 106.019417) (end 117.602 108.746427) (width 0.3048) (layer F.Cu) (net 18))
 (segment (start 117.602 108.746427) (end 117.602 113.538) (width 0.3048) (layer F.Cu) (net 18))
 (segment (start 113.03 118.11) (end 117.856 113.284) (width 0.2032) (layer B.Cu) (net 18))
 (segment (start 117.856 107.369893) (end 121.040301 104.185592) (width 0.2032) (layer B.Cu) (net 18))
 (segment (start 117.856 113.284) (end 117.856 107.369893) (width 0.2032) (layer B.Cu) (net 18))
 (segment (start 126.905103 102.625305) (end 127.889 103.609202) (width 0.3048) (layer F.Cu) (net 9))
 (segment (start 130.81 102.87) (end 129.667 104.013) (width 0.3048) (layer F.Cu) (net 9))
 (segment (start 128.292798 104.013) (end 127.889 103.609202) (width 0.3048) (layer F.Cu) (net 9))
 (segment (start 129.667 104.013) (end 128.292798 104.013) (width 0.3048) (layer F.Cu) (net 9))
 (segment (start 129.54 104.14) (end 130.81 102.87) (width 0.2032) (layer B.Cu) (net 9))
 (segment (start 124.841 102.064272) (end 126.916728 104.14) (width 0.2032) (layer B.Cu) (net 9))
 (segment (start 126.916728 104.14) (end 129.54 104.14) (width 0.2032) (layer B.Cu) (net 9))
 (segment (start 125.603 115.443) (end 130.81 120.65) (width 0.3048) (layer F.Cu) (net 16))
 (segment (start 125.603 109.22) (end 125.603 115.443) (width 0.3048) (layer F.Cu) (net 16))
 (segment (start 122.945305 106.585103) (end 122.968103 106.585103) (width 0.3048) (layer F.Cu) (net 16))
 (segment (start 122.968103 106.585103) (end 125.603 109.22) (width 0.3048) (layer F.Cu) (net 16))
 (segment (start 124.333 114.173) (end 130.81 120.65) (width 0.2032) (layer B.Cu) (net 16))
 (segment (start 124.333 106.50602) (end 122.366126 104.539146) (width 0.2032) (layer B.Cu) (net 16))
 (segment (start 124.333 114.173) (end 124.333 106.50602) (width 0.2032) (layer B.Cu) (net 16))
 (segment (start 126.365 113.665) (end 130.81 118.11) (width 0.3048) (layer F.Cu) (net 15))
 (segment (start 123.51099 106.019417) (end 126.365 108.873427) (width 0.3048) (layer F.Cu) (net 15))
 (segment (start 126.365 108.873427) (end 126.365 113.665) (width 0.3048) (layer F.Cu) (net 15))
 (segment (start 122.719679 104.185592) (end 125.222 106.687913) (width 0.2032) (layer B.Cu) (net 15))
 (segment (start 125.222 112.522) (end 130.81 118.11) (width 0.2032) (layer B.Cu) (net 15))
 (segment (start 125.222 106.687913) (end 125.222 112.522) (width 0.2032) (layer B.Cu) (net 15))
 (segment (start 127.254 112.014) (end 130.81 115.57) (width 0.3048) (layer F.Cu) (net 14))
 (segment (start 127.254 108.712) (end 127.254 112.014) (width 0.3048) (layer F.Cu) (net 14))
 (segment (start 124.713071 106.171071) (end 127.254 108.712) (width 0.3048) (layer F.Cu) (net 14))
 (segment (start 124.076676 105.453732) (end 124.713071 106.090127) (width 0.3048) (layer F.Cu) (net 14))
 (segment (start 124.713071 106.090127) (end 124.713071 106.171071) (width 0.3048) (layer F.Cu) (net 14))
 (segment (start 126.238 110.998) (end 130.81 115.57) (width 0.2032) (layer B.Cu) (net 14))
 (segment (start 123.073233 103.832039) (end 126.238 106.996806) (width 0.2032) (layer B.Cu) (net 14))
 (segment (start 126.238 106.996806) (end 126.238 110.998) (width 0.2032) (layer B.Cu) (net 14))
 (segment (start 128.143 110.363) (end 130.81 113.03) (width 0.3048) (layer F.Cu) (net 13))
 (segment (start 128.143 108.458) (end 128.143 110.363) (width 0.3048) (layer F.Cu) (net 13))
 (segment (start 125.278756 105.593756) (end 128.143 108.458) (width 0.3048) (layer F.Cu) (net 13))
 (segment (start 124.642361 104.888047) (end 125.278756 105.524442) (width 0.3048) (layer F.Cu) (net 13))
 (segment (start 125.278756 105.524442) (end 125.278756 105.593756) (width 0.3048) (layer F.Cu) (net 13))
 (segment (start 129.960001 112.180001) (end 130.81 113.03) (width 0.2032) (layer B.Cu) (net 13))
 (segment (start 127.381 109.601) (end 129.960001 112.180001) (width 0.2032) (layer B.Cu) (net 13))
 (segment (start 123.426786 103.478485) (end 127.381 107.432699) (width 0.2032) (layer B.Cu) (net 13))
 (segment (start 127.381 107.432699) (end 127.381 109.601) (width 0.2032) (layer B.Cu) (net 13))
 (segment (start 128.9685 108.6485) (end 130.81 110.49) (width 0.3048) (layer F.Cu) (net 12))
 (segment (start 125.208047 104.322361) (end 128.9685 108.082814) (width 0.3048) (layer F.Cu) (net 12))
 (segment (start 128.9685 108.082814) (end 128.9685 108.6485) (width 0.3048) (layer F.Cu) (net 12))
 (segment (start 130.81 110.154593) (end 130.81 110.49) (width 0.2032) (layer B.Cu) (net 12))
 (segment (start 128.524 108.204) (end 130.81 110.49) (width 0.2032) (layer B.Cu) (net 12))
 (segment (start 123.780339 103.124932) (end 128.524 107.868593) (width 0.2032) (layer B.Cu) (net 12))
 (segment (start 128.524 107.868593) (end 128.524 108.204) (width 0.2032) (layer B.Cu) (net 12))
 (segment (start 126.410127 104.393071) (end 125.773732 103.756676) (width 0.3048) (layer F.Cu) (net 11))
 (segment (start 129.117057 107.100001) (end 126.410127 104.393071) (width 0.3048) (layer F.Cu) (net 11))
 (segment (start 129.960001 107.100001) (end 129.117057 107.100001) (width 0.3048) (layer F.Cu) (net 11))
 (segment (start 130.81 107.95) (end 129.960001 107.100001) (width 0.3048) (layer F.Cu) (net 11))
 (segment (start 129.312514 107.95) (end 130.81 107.95) (width 0.2032) (layer B.Cu) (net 11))
 (segment (start 124.133893 102.771379) (end 129.312514 107.95) (width 0.2032) (layer B.Cu) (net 11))
 (segment (start 128.558427 105.41) (end 130.81 105.41) (width 0.3048) (layer F.Cu) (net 10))
 (segment (start 126.339417 103.19099) (end 128.558427 105.41) (width 0.3048) (layer F.Cu) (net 10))
 (segment (start 127.479621 105.41) (end 130.81 105.41) (width 0.2032) (layer B.Cu) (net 10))
 (segment (start 124.487446 102.417825) (end 127.479621 105.41) (width 0.2032) (layer B.Cu) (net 10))
 (segment (start 129.960001 83.399999) (end 130.81 82.55) (width 0.3048) (layer F.Cu) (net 1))
 (segment (start 126.111 87.249) (end 129.960001 83.399999) (width 0.3048) (layer F.Cu) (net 1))
 (segment (start 122.945305 96.614897) (end 126.111 93.449202) (width 0.3048) (layer F.Cu) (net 1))
 (segment (start 126.111 93.449202) (end 126.111 87.249) (width 0.3048) (layer F.Cu) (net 1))
 (segment (start 122.366126 98.34035) (end 125.349 95.357476) (width 0.2032) (layer B.Cu) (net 1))
 (segment (start 122.366126 98.617126) (end 122.366126 98.34035) (width 0.2032) (layer B.Cu) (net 1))
 (segment (start 125.349 88.011) (end 130.81 82.55) (width 0.2032) (layer B.Cu) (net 1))
 (segment (start 125.349 95.357476) (end 125.349 88.011) (width 0.2032) (layer B.Cu) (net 1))
 (segment (start 129.667 99.187) (end 130.81 100.33) (width 0.3048) (layer F.Cu) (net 8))
 (segment (start 126.905103 100.574695) (end 128.292798 99.187) (width 0.3048) (layer F.Cu) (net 8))
 (segment (start 128.292798 99.187) (end 129.667 99.187) (width 0.3048) (layer F.Cu) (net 8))
 (segment (start 129.286 98.806) (end 130.81 100.33) (width 0.2032) (layer B.Cu) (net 8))
 (segment (start 124.841 101.092) (end 127.127 98.806) (width 0.2032) (layer B.Cu) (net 8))
 (segment (start 127.127 98.806) (end 129.286 98.806) (width 0.2032) (layer B.Cu) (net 8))
 (segment (start 128.558427 97.79) (end 130.81 97.79) (width 0.3048) (layer F.Cu) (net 7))
 (segment (start 126.339417 100.00901) (end 128.558427 97.79) (width 0.3048) (layer F.Cu) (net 7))
 (segment (start 127.435893 97.79) (end 130.81 97.79) (width 0.2032) (layer B.Cu) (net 7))
 (segment (start 124.487446 100.738447) (end 127.435893 97.79) (width 0.2032) (layer B.Cu) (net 7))
 (segment (start 129.967056 95.25) (end 130.81 95.25) (width 0.3048) (layer F.Cu) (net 6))
 (segment (start 125.773732 99.443324) (end 129.967056 95.25) (width 0.3048) (layer F.Cu) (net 6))
 (segment (start 129.54 96.52) (end 130.81 95.25) (width 0.2032) (layer B.Cu) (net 6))
 (segment (start 124.133893 100.384893) (end 127.998786 96.52) (width 0.2032) (layer B.Cu) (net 6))
 (segment (start 127.998786 96.52) (end 129.54 96.52) (width 0.2032) (layer B.Cu) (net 6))
 (segment (start 129.159 94.361) (end 130.81 92.71) (width 0.3048) (layer F.Cu) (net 5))
 (segment (start 125.208047 98.877639) (end 129.159 94.926686) (width 0.3048) (layer F.Cu) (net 5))
 (segment (start 129.159 94.926686) (end 129.159 94.361) (width 0.3048) (layer F.Cu) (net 5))
 (segment (start 130.81 93.001679) (end 130.81 92.71) (width 0.2032) (layer B.Cu) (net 5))
 (segment (start 123.780339 100.03134) (end 130.81 93.001679) (width 0.2032) (layer B.Cu) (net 5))
 (segment (start 128.397 92.583) (end 130.81 90.17) (width 0.3048) (layer F.Cu) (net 4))
 (segment (start 124.642361 98.311953) (end 128.397 94.557314) (width 0.3048) (layer F.Cu) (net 4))
 (segment (start 128.397 94.557314) (end 128.397 92.583) (width 0.3048) (layer F.Cu) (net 4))
 (segment (start 129.960001 91.019999) (end 130.81 90.17) (width 0.2032) (layer B.Cu) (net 4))
 (segment (start 128.016 92.964) (end 129.960001 91.019999) (width 0.2032) (layer B.Cu) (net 4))
 (segment (start 123.426786 99.677787) (end 128.016 95.088573) (width 0.2032) (layer B.Cu) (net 4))
 (segment (start 128.016 95.088573) (end 128.016 92.964) (width 0.2032) (layer B.Cu) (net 4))
 (segment (start 127.635 90.805) (end 130.81 87.63) (width 0.3048) (layer F.Cu) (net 3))
 (segment (start 124.076676 97.746268) (end 127.635 94.187944) (width 0.3048) (layer F.Cu) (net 3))
 (segment (start 127.635 94.187944) (end 127.635 90.805) (width 0.3048) (layer F.Cu) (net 3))
 (segment (start 129.960001 88.479999) (end 130.81 87.63) (width 0.2032) (layer B.Cu) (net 3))
 (segment (start 127.127 91.313) (end 129.960001 88.479999) (width 0.2032) (layer B.Cu) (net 3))
 (segment (start 123.073233 99.324233) (end 127.127 95.270466) (width 0.2032) (layer B.Cu) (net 3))
 (segment (start 127.127 95.270466) (end 127.127 91.313) (width 0.2032) (layer B.Cu) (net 3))
 (segment (start 126.873 89.027) (end 130.81 85.09) (width 0.3048) (layer F.Cu) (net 2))
 (segment (start 123.51099 97.180583) (end 126.873 93.818573) (width 0.3048) (layer F.Cu) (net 2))
 (segment (start 126.873 93.818573) (end 126.873 89.027) (width 0.3048) (layer F.Cu) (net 2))
 (segment (start 129.960001 85.939999) (end 130.81 85.09) (width 0.2032) (layer B.Cu) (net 2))
 (segment (start 126.365 89.535) (end 129.960001 85.939999) (width 0.2032) (layer B.Cu) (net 2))
 (segment (start 122.719679 98.97068) (end 126.365 95.325359) (width 0.2032) (layer B.Cu) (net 2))
 (segment (start 126.365 95.325359) (end 126.365 89.535) (width 0.2032) (layer B.Cu) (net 2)))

